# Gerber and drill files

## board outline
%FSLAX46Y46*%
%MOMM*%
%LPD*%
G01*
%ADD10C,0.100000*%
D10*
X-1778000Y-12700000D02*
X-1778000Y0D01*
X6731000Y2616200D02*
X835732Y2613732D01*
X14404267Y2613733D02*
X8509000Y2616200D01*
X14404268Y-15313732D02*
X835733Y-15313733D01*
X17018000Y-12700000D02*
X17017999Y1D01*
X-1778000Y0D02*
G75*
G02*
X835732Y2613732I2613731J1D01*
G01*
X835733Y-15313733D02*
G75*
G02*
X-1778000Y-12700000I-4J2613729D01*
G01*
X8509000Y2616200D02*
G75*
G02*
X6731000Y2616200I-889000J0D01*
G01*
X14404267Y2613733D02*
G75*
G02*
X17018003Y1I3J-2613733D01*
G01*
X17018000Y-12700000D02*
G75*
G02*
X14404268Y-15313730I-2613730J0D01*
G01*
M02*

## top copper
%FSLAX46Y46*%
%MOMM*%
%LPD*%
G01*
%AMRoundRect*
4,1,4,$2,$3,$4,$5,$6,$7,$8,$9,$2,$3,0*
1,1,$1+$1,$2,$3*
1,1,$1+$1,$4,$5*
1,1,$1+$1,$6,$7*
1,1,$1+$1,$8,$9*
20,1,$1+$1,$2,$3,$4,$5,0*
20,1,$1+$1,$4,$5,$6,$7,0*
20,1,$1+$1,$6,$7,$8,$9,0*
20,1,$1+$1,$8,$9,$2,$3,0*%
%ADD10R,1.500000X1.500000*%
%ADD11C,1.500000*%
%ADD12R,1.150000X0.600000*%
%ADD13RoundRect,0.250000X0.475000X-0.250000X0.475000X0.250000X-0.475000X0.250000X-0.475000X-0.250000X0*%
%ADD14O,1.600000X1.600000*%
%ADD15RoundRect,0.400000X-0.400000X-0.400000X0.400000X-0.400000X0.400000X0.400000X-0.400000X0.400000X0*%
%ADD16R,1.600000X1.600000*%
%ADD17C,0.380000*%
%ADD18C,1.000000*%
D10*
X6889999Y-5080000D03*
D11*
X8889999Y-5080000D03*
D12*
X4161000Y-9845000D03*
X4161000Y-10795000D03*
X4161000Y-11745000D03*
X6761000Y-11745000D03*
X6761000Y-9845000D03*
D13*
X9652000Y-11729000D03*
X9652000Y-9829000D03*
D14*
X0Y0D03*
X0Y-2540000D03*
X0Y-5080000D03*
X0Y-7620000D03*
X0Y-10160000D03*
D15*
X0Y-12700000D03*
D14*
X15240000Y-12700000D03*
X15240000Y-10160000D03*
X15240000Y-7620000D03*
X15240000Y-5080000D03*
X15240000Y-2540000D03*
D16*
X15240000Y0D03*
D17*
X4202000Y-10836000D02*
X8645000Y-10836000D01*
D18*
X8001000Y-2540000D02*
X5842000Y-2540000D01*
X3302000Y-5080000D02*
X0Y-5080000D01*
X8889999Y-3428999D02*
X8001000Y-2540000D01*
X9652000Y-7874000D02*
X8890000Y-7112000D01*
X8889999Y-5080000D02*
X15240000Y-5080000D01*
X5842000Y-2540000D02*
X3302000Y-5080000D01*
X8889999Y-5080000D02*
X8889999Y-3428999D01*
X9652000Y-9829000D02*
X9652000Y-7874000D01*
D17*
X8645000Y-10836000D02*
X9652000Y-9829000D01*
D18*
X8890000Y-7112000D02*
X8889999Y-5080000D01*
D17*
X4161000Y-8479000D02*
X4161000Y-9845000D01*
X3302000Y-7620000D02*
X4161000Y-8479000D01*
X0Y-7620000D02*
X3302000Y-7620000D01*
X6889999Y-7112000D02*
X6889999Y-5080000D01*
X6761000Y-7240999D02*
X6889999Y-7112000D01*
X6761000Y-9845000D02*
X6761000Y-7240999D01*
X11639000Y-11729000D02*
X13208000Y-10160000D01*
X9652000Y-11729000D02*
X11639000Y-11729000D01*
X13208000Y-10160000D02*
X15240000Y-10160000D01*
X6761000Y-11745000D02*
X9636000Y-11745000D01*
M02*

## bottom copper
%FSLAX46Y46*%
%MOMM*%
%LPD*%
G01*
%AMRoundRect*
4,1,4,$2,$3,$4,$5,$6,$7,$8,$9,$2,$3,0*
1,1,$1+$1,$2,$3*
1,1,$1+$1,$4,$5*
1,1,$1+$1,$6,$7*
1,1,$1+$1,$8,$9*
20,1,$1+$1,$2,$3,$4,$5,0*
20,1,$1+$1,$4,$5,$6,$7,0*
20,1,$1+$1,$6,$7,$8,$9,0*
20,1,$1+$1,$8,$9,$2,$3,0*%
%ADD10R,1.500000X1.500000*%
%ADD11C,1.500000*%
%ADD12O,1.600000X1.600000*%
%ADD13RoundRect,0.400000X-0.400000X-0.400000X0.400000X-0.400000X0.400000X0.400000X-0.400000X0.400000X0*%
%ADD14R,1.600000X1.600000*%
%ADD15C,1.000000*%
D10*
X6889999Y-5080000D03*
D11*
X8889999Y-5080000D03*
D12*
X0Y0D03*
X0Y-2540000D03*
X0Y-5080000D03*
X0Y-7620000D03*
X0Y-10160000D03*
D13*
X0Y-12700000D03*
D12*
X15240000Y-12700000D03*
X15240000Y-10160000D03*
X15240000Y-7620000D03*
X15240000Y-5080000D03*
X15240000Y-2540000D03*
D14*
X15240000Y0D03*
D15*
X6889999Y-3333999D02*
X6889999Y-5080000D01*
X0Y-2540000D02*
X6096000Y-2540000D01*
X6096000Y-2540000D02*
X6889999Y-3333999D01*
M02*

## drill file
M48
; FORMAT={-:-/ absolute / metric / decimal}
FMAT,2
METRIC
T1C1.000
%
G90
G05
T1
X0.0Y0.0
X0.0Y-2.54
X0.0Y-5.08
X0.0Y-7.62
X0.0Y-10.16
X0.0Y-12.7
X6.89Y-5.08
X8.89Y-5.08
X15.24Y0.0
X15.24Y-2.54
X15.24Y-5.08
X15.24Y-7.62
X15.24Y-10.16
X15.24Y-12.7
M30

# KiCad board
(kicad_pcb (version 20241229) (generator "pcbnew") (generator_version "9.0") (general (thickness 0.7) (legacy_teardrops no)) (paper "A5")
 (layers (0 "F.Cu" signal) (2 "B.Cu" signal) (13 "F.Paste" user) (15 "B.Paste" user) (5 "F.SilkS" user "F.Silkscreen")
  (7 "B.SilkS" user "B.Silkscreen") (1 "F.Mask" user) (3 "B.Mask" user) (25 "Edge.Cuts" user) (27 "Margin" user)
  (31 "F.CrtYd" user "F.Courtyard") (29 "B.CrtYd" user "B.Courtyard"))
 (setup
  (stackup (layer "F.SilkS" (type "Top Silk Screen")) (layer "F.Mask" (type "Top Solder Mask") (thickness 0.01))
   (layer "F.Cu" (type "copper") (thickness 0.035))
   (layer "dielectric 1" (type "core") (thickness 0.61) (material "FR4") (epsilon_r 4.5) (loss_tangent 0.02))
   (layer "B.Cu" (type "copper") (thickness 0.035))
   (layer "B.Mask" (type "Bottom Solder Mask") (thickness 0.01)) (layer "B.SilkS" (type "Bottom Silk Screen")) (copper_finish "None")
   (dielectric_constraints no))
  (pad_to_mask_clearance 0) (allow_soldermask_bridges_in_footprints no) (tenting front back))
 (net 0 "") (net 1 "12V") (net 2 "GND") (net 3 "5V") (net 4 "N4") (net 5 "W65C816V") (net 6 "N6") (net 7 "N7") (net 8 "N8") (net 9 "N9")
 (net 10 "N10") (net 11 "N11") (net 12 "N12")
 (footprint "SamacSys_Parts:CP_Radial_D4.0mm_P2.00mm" (layer "F.Cu") (at 6.889999 5.08)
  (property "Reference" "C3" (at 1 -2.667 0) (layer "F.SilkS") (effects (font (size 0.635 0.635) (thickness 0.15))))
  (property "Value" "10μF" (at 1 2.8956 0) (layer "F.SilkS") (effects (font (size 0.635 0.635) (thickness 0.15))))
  (pad "1" thru_hole rect (at 0 0) (size 1.5 1.5) (drill 1) (layers "*.Cu" "*.Mask") (remove_unused_layers no) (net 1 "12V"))
  (pad "2" thru_hole circle (at 2 0) (size 1.5 1.5) (drill 1) (layers "*.Cu" "*.Mask") (remove_unused_layers no) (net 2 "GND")))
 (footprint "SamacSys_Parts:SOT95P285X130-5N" (layer "F.Cu") (at 5.461 10.795)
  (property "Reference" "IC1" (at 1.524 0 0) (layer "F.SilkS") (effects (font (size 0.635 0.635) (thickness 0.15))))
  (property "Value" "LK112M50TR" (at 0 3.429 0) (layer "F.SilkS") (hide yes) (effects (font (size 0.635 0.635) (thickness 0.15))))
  (pad "1" smd rect (at -1.3 -0.95 90) (size 0.6 1.15) (layers "F.Cu" "F.Mask" "F.Paste") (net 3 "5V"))
  (pad "2" smd rect (at -1.3 0 90) (size 0.6 1.15) (layers "F.Cu" "F.Mask" "F.Paste") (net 2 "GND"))
  (pad "3" smd rect (at -1.3 0.95 90) (size 0.6 1.15) (layers "F.Cu" "F.Mask" "F.Paste") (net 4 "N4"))
  (pad "4" smd rect (at 1.3 0.95 90) (size 0.6 1.15) (layers "F.Cu" "F.Mask" "F.Paste") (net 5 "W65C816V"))
  (pad "5" smd rect (at 1.3 -0.95 90) (size 0.6 1.15) (layers "F.Cu" "F.Mask" "F.Paste") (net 1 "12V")))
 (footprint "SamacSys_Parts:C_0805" (layer "F.Cu") (at 9.652 10.795)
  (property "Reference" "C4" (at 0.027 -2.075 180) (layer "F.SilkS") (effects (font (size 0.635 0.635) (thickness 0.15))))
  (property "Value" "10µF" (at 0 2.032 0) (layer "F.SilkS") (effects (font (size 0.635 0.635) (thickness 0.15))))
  (pad "1" smd roundrect (at 0 0.934 90) (size 1 1.45) (layers "F.Cu" "F.Mask" "F.Paste") (roundrect_rratio 0.25) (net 5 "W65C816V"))
  (pad "2" smd roundrect (at 0 -0.966 90) (size 1 1.45) (layers "F.Cu" "F.Mask" "F.Paste") (roundrect_rratio 0.25) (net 2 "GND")))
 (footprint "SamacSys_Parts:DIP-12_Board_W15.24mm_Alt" (layer "F.Cu") (at 0 0)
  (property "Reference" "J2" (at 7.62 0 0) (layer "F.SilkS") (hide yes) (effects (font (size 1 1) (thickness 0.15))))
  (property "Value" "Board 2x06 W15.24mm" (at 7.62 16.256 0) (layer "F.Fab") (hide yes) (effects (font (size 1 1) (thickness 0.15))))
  (fp_line (start -1.778 12.7) (end -1.778 0) (stroke (width 0.1) (type solid)) (layer "Edge.Cuts"))
  (fp_line (start 6.731 -2.6162) (end 0.835732 -2.613732) (stroke (width 0.1) (type solid)) (layer "Edge.Cuts"))
  (fp_line (start 14.404267 -2.613733) (end 8.509 -2.6162) (stroke (width 0.1) (type solid)) (layer "Edge.Cuts"))
  (fp_line (start 14.404268 15.313732) (end 0.835733 15.313733) (stroke (width 0.1) (type solid)) (layer "Edge.Cuts"))
  (fp_line (start 17.018 12.7) (end 17.017999 -0.000001) (stroke (width 0.1) (type solid)) (layer "Edge.Cuts"))
  (fp_arc (start -1.778 0) (mid -1.012456 -1.848188) (end 0.835732 -2.613732) (stroke (width 0.1) (type solid)) (layer "Edge.Cuts"))
  (fp_arc (start 0.835733 15.313733) (mid -1.012457 14.548189) (end -1.778 12.7) (stroke (width 0.1) (type solid)) (layer "Edge.Cuts"))
  (fp_arc (start 8.509 -2.6162) (mid 7.62 -1.7272) (end 6.731 -2.6162) (stroke (width 0.1) (type default)) (layer "Edge.Cuts"))
  (fp_arc (start 14.404267 -2.613733) (mid 16.252455 -1.848189) (end 17.017999 -0.000001) (stroke (width 0.1) (type solid))
   (layer "Edge.Cuts"))
  (fp_arc (start 17.018 12.7) (mid 16.252456 14.548187) (end 14.404268 15.313732) (stroke (width 0.1) (type solid)) (layer "Edge.Cuts"))
  (pad "1" thru_hole oval (at 0 0 180) (size 1.6 1.6) (drill 1) (layers "*.Cu" "*.Mask") (remove_unused_layers no) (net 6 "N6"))
  (pad "2" thru_hole oval (at 0 2.54) (size 1.6 1.6) (drill 1) (layers "*.Cu" "*.Mask") (remove_unused_layers no) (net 1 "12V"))
  (pad "3" thru_hole oval (at 0 5.08) (size 1.6 1.6) (drill 1) (layers "*.Cu" "*.Mask") (remove_unused_layers no) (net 2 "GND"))
  (pad "4" thru_hole oval (at 0 7.62 180) (size 1.6 1.6) (drill 1) (layers "*.Cu" "*.Mask") (remove_unused_layers no) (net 3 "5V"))
  (pad "5" thru_hole oval (at 0 10.16) (size 1.6 1.6) (drill 1) (layers "*.Cu" "*.Mask") (remove_unused_layers no) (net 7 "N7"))
  (pad "6" thru_hole roundrect (at 0 12.7) (size 1.6 1.6) (drill 1) (layers "*.Cu" "*.Mask") (remove_unused_layers no)
   (roundrect_rratio 0.25) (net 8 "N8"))
  (pad "7" thru_hole oval (at 15.24 12.7 180) (size 1.6 1.6) (drill 1) (layers "*.Cu" "*.Mask") (remove_unused_layers no) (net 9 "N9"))
  (pad "8" thru_hole oval (at 15.24 10.16 180) (size 1.6 1.6) (drill 1) (layers "*.Cu" "*.Mask") (remove_unused_layers no)
   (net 5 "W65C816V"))
  (pad "9" thru_hole oval (at 15.24 7.62 180) (size 1.6 1.6) (drill 1) (layers "*.Cu" "*.Mask") (remove_unused_layers no) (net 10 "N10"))
  (pad "10" thru_hole oval (at 15.24 5.08) (size 1.6 1.6) (drill 1) (layers "*.Cu" "*.Mask") (remove_unused_layers no) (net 2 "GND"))
  (pad "11" thru_hole oval (at 15.24 2.54) (size 1.6 1.6) (drill 1) (layers "*.Cu" "*.Mask") (remove_unused_layers no) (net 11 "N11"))
  (pad "12" thru_hole rect (at 15.24 0) (size 1.6 1.6) (drill 1) (layers "*.Cu" "*.Mask") (remove_unused_layers no) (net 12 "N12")))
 (segment (start 4.202 10.836) (end 8.645 10.836) (width 0.38) (layer "F.Cu") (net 2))
 (segment (start 8.001 2.54) (end 5.842 2.54) (width 1) (layer "F.Cu") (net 2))
 (segment (start 3.302 5.08) (end 0 5.08) (width 1) (layer "F.Cu") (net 2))
 (segment (start 8.889999 3.428999) (end 8.001 2.54) (width 1) (layer "F.Cu") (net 2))
 (segment (start 9.652 7.874) (end 8.89 7.112) (width 1) (layer "F.Cu") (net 2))
 (segment (start 8.889999 5.08) (end 15.24 5.08) (width 1) (layer "F.Cu") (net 2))
 (segment (start 5.842 2.54) (end 3.302 5.08) (width 1) (layer "F.Cu") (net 2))
 (segment (start 8.889999 5.08) (end 8.889999 3.428999) (width 1) (layer "F.Cu") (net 2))
 (segment (start 9.652 9.829) (end 9.652 7.874) (width 1) (layer "F.Cu") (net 2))
 (segment (start 8.645 10.836) (end 9.652 9.829) (width 0.38) (layer "F.Cu") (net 2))
 (segment (start 8.89 7.112) (end 8.889999 5.08) (width 1) (layer "F.Cu") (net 2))
 (segment (start 4.161 8.479) (end 4.161 9.845) (width 0.38) (layer "F.Cu") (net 3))
 (segment (start 3.302 7.62) (end 4.161 8.479) (width 0.38) (layer "F.Cu") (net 3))
 (segment (start 0 7.62) (end 3.302 7.62) (width 0.38) (layer "F.Cu") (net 3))
 (segment (start 6.889999 7.112) (end 6.889999 5.08) (width 0.38) (layer "F.Cu") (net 1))
 (segment (start 6.761 7.240999) (end 6.889999 7.112) (width 0.38) (layer "F.Cu") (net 1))
 (segment (start 6.761 9.845) (end 6.761 7.240999) (width 0.38) (layer "F.Cu") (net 1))
 (segment (start 6.889999 3.333999) (end 6.889999 5.08) (width 1) (layer "B.Cu") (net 1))
 (segment (start 0 2.54) (end 6.096 2.54) (width 1) (layer "B.Cu") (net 1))
 (segment (start 6.096 2.54) (end 6.889999 3.333999) (width 1) (layer "B.Cu") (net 1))
 (segment (start 11.639 11.729) (end 13.208 10.16) (width 0.38) (layer "F.Cu") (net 5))
 (segment (start 9.652 11.729) (end 11.639 11.729) (width 0.38) (layer "F.Cu") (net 5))
 (segment (start 13.208 10.16) (end 15.24 10.16) (width 0.38) (layer "F.Cu") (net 5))
 (segment (start 6.761 11.745) (end 9.636 11.745) (width 0.38) (layer "F.Cu") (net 5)))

